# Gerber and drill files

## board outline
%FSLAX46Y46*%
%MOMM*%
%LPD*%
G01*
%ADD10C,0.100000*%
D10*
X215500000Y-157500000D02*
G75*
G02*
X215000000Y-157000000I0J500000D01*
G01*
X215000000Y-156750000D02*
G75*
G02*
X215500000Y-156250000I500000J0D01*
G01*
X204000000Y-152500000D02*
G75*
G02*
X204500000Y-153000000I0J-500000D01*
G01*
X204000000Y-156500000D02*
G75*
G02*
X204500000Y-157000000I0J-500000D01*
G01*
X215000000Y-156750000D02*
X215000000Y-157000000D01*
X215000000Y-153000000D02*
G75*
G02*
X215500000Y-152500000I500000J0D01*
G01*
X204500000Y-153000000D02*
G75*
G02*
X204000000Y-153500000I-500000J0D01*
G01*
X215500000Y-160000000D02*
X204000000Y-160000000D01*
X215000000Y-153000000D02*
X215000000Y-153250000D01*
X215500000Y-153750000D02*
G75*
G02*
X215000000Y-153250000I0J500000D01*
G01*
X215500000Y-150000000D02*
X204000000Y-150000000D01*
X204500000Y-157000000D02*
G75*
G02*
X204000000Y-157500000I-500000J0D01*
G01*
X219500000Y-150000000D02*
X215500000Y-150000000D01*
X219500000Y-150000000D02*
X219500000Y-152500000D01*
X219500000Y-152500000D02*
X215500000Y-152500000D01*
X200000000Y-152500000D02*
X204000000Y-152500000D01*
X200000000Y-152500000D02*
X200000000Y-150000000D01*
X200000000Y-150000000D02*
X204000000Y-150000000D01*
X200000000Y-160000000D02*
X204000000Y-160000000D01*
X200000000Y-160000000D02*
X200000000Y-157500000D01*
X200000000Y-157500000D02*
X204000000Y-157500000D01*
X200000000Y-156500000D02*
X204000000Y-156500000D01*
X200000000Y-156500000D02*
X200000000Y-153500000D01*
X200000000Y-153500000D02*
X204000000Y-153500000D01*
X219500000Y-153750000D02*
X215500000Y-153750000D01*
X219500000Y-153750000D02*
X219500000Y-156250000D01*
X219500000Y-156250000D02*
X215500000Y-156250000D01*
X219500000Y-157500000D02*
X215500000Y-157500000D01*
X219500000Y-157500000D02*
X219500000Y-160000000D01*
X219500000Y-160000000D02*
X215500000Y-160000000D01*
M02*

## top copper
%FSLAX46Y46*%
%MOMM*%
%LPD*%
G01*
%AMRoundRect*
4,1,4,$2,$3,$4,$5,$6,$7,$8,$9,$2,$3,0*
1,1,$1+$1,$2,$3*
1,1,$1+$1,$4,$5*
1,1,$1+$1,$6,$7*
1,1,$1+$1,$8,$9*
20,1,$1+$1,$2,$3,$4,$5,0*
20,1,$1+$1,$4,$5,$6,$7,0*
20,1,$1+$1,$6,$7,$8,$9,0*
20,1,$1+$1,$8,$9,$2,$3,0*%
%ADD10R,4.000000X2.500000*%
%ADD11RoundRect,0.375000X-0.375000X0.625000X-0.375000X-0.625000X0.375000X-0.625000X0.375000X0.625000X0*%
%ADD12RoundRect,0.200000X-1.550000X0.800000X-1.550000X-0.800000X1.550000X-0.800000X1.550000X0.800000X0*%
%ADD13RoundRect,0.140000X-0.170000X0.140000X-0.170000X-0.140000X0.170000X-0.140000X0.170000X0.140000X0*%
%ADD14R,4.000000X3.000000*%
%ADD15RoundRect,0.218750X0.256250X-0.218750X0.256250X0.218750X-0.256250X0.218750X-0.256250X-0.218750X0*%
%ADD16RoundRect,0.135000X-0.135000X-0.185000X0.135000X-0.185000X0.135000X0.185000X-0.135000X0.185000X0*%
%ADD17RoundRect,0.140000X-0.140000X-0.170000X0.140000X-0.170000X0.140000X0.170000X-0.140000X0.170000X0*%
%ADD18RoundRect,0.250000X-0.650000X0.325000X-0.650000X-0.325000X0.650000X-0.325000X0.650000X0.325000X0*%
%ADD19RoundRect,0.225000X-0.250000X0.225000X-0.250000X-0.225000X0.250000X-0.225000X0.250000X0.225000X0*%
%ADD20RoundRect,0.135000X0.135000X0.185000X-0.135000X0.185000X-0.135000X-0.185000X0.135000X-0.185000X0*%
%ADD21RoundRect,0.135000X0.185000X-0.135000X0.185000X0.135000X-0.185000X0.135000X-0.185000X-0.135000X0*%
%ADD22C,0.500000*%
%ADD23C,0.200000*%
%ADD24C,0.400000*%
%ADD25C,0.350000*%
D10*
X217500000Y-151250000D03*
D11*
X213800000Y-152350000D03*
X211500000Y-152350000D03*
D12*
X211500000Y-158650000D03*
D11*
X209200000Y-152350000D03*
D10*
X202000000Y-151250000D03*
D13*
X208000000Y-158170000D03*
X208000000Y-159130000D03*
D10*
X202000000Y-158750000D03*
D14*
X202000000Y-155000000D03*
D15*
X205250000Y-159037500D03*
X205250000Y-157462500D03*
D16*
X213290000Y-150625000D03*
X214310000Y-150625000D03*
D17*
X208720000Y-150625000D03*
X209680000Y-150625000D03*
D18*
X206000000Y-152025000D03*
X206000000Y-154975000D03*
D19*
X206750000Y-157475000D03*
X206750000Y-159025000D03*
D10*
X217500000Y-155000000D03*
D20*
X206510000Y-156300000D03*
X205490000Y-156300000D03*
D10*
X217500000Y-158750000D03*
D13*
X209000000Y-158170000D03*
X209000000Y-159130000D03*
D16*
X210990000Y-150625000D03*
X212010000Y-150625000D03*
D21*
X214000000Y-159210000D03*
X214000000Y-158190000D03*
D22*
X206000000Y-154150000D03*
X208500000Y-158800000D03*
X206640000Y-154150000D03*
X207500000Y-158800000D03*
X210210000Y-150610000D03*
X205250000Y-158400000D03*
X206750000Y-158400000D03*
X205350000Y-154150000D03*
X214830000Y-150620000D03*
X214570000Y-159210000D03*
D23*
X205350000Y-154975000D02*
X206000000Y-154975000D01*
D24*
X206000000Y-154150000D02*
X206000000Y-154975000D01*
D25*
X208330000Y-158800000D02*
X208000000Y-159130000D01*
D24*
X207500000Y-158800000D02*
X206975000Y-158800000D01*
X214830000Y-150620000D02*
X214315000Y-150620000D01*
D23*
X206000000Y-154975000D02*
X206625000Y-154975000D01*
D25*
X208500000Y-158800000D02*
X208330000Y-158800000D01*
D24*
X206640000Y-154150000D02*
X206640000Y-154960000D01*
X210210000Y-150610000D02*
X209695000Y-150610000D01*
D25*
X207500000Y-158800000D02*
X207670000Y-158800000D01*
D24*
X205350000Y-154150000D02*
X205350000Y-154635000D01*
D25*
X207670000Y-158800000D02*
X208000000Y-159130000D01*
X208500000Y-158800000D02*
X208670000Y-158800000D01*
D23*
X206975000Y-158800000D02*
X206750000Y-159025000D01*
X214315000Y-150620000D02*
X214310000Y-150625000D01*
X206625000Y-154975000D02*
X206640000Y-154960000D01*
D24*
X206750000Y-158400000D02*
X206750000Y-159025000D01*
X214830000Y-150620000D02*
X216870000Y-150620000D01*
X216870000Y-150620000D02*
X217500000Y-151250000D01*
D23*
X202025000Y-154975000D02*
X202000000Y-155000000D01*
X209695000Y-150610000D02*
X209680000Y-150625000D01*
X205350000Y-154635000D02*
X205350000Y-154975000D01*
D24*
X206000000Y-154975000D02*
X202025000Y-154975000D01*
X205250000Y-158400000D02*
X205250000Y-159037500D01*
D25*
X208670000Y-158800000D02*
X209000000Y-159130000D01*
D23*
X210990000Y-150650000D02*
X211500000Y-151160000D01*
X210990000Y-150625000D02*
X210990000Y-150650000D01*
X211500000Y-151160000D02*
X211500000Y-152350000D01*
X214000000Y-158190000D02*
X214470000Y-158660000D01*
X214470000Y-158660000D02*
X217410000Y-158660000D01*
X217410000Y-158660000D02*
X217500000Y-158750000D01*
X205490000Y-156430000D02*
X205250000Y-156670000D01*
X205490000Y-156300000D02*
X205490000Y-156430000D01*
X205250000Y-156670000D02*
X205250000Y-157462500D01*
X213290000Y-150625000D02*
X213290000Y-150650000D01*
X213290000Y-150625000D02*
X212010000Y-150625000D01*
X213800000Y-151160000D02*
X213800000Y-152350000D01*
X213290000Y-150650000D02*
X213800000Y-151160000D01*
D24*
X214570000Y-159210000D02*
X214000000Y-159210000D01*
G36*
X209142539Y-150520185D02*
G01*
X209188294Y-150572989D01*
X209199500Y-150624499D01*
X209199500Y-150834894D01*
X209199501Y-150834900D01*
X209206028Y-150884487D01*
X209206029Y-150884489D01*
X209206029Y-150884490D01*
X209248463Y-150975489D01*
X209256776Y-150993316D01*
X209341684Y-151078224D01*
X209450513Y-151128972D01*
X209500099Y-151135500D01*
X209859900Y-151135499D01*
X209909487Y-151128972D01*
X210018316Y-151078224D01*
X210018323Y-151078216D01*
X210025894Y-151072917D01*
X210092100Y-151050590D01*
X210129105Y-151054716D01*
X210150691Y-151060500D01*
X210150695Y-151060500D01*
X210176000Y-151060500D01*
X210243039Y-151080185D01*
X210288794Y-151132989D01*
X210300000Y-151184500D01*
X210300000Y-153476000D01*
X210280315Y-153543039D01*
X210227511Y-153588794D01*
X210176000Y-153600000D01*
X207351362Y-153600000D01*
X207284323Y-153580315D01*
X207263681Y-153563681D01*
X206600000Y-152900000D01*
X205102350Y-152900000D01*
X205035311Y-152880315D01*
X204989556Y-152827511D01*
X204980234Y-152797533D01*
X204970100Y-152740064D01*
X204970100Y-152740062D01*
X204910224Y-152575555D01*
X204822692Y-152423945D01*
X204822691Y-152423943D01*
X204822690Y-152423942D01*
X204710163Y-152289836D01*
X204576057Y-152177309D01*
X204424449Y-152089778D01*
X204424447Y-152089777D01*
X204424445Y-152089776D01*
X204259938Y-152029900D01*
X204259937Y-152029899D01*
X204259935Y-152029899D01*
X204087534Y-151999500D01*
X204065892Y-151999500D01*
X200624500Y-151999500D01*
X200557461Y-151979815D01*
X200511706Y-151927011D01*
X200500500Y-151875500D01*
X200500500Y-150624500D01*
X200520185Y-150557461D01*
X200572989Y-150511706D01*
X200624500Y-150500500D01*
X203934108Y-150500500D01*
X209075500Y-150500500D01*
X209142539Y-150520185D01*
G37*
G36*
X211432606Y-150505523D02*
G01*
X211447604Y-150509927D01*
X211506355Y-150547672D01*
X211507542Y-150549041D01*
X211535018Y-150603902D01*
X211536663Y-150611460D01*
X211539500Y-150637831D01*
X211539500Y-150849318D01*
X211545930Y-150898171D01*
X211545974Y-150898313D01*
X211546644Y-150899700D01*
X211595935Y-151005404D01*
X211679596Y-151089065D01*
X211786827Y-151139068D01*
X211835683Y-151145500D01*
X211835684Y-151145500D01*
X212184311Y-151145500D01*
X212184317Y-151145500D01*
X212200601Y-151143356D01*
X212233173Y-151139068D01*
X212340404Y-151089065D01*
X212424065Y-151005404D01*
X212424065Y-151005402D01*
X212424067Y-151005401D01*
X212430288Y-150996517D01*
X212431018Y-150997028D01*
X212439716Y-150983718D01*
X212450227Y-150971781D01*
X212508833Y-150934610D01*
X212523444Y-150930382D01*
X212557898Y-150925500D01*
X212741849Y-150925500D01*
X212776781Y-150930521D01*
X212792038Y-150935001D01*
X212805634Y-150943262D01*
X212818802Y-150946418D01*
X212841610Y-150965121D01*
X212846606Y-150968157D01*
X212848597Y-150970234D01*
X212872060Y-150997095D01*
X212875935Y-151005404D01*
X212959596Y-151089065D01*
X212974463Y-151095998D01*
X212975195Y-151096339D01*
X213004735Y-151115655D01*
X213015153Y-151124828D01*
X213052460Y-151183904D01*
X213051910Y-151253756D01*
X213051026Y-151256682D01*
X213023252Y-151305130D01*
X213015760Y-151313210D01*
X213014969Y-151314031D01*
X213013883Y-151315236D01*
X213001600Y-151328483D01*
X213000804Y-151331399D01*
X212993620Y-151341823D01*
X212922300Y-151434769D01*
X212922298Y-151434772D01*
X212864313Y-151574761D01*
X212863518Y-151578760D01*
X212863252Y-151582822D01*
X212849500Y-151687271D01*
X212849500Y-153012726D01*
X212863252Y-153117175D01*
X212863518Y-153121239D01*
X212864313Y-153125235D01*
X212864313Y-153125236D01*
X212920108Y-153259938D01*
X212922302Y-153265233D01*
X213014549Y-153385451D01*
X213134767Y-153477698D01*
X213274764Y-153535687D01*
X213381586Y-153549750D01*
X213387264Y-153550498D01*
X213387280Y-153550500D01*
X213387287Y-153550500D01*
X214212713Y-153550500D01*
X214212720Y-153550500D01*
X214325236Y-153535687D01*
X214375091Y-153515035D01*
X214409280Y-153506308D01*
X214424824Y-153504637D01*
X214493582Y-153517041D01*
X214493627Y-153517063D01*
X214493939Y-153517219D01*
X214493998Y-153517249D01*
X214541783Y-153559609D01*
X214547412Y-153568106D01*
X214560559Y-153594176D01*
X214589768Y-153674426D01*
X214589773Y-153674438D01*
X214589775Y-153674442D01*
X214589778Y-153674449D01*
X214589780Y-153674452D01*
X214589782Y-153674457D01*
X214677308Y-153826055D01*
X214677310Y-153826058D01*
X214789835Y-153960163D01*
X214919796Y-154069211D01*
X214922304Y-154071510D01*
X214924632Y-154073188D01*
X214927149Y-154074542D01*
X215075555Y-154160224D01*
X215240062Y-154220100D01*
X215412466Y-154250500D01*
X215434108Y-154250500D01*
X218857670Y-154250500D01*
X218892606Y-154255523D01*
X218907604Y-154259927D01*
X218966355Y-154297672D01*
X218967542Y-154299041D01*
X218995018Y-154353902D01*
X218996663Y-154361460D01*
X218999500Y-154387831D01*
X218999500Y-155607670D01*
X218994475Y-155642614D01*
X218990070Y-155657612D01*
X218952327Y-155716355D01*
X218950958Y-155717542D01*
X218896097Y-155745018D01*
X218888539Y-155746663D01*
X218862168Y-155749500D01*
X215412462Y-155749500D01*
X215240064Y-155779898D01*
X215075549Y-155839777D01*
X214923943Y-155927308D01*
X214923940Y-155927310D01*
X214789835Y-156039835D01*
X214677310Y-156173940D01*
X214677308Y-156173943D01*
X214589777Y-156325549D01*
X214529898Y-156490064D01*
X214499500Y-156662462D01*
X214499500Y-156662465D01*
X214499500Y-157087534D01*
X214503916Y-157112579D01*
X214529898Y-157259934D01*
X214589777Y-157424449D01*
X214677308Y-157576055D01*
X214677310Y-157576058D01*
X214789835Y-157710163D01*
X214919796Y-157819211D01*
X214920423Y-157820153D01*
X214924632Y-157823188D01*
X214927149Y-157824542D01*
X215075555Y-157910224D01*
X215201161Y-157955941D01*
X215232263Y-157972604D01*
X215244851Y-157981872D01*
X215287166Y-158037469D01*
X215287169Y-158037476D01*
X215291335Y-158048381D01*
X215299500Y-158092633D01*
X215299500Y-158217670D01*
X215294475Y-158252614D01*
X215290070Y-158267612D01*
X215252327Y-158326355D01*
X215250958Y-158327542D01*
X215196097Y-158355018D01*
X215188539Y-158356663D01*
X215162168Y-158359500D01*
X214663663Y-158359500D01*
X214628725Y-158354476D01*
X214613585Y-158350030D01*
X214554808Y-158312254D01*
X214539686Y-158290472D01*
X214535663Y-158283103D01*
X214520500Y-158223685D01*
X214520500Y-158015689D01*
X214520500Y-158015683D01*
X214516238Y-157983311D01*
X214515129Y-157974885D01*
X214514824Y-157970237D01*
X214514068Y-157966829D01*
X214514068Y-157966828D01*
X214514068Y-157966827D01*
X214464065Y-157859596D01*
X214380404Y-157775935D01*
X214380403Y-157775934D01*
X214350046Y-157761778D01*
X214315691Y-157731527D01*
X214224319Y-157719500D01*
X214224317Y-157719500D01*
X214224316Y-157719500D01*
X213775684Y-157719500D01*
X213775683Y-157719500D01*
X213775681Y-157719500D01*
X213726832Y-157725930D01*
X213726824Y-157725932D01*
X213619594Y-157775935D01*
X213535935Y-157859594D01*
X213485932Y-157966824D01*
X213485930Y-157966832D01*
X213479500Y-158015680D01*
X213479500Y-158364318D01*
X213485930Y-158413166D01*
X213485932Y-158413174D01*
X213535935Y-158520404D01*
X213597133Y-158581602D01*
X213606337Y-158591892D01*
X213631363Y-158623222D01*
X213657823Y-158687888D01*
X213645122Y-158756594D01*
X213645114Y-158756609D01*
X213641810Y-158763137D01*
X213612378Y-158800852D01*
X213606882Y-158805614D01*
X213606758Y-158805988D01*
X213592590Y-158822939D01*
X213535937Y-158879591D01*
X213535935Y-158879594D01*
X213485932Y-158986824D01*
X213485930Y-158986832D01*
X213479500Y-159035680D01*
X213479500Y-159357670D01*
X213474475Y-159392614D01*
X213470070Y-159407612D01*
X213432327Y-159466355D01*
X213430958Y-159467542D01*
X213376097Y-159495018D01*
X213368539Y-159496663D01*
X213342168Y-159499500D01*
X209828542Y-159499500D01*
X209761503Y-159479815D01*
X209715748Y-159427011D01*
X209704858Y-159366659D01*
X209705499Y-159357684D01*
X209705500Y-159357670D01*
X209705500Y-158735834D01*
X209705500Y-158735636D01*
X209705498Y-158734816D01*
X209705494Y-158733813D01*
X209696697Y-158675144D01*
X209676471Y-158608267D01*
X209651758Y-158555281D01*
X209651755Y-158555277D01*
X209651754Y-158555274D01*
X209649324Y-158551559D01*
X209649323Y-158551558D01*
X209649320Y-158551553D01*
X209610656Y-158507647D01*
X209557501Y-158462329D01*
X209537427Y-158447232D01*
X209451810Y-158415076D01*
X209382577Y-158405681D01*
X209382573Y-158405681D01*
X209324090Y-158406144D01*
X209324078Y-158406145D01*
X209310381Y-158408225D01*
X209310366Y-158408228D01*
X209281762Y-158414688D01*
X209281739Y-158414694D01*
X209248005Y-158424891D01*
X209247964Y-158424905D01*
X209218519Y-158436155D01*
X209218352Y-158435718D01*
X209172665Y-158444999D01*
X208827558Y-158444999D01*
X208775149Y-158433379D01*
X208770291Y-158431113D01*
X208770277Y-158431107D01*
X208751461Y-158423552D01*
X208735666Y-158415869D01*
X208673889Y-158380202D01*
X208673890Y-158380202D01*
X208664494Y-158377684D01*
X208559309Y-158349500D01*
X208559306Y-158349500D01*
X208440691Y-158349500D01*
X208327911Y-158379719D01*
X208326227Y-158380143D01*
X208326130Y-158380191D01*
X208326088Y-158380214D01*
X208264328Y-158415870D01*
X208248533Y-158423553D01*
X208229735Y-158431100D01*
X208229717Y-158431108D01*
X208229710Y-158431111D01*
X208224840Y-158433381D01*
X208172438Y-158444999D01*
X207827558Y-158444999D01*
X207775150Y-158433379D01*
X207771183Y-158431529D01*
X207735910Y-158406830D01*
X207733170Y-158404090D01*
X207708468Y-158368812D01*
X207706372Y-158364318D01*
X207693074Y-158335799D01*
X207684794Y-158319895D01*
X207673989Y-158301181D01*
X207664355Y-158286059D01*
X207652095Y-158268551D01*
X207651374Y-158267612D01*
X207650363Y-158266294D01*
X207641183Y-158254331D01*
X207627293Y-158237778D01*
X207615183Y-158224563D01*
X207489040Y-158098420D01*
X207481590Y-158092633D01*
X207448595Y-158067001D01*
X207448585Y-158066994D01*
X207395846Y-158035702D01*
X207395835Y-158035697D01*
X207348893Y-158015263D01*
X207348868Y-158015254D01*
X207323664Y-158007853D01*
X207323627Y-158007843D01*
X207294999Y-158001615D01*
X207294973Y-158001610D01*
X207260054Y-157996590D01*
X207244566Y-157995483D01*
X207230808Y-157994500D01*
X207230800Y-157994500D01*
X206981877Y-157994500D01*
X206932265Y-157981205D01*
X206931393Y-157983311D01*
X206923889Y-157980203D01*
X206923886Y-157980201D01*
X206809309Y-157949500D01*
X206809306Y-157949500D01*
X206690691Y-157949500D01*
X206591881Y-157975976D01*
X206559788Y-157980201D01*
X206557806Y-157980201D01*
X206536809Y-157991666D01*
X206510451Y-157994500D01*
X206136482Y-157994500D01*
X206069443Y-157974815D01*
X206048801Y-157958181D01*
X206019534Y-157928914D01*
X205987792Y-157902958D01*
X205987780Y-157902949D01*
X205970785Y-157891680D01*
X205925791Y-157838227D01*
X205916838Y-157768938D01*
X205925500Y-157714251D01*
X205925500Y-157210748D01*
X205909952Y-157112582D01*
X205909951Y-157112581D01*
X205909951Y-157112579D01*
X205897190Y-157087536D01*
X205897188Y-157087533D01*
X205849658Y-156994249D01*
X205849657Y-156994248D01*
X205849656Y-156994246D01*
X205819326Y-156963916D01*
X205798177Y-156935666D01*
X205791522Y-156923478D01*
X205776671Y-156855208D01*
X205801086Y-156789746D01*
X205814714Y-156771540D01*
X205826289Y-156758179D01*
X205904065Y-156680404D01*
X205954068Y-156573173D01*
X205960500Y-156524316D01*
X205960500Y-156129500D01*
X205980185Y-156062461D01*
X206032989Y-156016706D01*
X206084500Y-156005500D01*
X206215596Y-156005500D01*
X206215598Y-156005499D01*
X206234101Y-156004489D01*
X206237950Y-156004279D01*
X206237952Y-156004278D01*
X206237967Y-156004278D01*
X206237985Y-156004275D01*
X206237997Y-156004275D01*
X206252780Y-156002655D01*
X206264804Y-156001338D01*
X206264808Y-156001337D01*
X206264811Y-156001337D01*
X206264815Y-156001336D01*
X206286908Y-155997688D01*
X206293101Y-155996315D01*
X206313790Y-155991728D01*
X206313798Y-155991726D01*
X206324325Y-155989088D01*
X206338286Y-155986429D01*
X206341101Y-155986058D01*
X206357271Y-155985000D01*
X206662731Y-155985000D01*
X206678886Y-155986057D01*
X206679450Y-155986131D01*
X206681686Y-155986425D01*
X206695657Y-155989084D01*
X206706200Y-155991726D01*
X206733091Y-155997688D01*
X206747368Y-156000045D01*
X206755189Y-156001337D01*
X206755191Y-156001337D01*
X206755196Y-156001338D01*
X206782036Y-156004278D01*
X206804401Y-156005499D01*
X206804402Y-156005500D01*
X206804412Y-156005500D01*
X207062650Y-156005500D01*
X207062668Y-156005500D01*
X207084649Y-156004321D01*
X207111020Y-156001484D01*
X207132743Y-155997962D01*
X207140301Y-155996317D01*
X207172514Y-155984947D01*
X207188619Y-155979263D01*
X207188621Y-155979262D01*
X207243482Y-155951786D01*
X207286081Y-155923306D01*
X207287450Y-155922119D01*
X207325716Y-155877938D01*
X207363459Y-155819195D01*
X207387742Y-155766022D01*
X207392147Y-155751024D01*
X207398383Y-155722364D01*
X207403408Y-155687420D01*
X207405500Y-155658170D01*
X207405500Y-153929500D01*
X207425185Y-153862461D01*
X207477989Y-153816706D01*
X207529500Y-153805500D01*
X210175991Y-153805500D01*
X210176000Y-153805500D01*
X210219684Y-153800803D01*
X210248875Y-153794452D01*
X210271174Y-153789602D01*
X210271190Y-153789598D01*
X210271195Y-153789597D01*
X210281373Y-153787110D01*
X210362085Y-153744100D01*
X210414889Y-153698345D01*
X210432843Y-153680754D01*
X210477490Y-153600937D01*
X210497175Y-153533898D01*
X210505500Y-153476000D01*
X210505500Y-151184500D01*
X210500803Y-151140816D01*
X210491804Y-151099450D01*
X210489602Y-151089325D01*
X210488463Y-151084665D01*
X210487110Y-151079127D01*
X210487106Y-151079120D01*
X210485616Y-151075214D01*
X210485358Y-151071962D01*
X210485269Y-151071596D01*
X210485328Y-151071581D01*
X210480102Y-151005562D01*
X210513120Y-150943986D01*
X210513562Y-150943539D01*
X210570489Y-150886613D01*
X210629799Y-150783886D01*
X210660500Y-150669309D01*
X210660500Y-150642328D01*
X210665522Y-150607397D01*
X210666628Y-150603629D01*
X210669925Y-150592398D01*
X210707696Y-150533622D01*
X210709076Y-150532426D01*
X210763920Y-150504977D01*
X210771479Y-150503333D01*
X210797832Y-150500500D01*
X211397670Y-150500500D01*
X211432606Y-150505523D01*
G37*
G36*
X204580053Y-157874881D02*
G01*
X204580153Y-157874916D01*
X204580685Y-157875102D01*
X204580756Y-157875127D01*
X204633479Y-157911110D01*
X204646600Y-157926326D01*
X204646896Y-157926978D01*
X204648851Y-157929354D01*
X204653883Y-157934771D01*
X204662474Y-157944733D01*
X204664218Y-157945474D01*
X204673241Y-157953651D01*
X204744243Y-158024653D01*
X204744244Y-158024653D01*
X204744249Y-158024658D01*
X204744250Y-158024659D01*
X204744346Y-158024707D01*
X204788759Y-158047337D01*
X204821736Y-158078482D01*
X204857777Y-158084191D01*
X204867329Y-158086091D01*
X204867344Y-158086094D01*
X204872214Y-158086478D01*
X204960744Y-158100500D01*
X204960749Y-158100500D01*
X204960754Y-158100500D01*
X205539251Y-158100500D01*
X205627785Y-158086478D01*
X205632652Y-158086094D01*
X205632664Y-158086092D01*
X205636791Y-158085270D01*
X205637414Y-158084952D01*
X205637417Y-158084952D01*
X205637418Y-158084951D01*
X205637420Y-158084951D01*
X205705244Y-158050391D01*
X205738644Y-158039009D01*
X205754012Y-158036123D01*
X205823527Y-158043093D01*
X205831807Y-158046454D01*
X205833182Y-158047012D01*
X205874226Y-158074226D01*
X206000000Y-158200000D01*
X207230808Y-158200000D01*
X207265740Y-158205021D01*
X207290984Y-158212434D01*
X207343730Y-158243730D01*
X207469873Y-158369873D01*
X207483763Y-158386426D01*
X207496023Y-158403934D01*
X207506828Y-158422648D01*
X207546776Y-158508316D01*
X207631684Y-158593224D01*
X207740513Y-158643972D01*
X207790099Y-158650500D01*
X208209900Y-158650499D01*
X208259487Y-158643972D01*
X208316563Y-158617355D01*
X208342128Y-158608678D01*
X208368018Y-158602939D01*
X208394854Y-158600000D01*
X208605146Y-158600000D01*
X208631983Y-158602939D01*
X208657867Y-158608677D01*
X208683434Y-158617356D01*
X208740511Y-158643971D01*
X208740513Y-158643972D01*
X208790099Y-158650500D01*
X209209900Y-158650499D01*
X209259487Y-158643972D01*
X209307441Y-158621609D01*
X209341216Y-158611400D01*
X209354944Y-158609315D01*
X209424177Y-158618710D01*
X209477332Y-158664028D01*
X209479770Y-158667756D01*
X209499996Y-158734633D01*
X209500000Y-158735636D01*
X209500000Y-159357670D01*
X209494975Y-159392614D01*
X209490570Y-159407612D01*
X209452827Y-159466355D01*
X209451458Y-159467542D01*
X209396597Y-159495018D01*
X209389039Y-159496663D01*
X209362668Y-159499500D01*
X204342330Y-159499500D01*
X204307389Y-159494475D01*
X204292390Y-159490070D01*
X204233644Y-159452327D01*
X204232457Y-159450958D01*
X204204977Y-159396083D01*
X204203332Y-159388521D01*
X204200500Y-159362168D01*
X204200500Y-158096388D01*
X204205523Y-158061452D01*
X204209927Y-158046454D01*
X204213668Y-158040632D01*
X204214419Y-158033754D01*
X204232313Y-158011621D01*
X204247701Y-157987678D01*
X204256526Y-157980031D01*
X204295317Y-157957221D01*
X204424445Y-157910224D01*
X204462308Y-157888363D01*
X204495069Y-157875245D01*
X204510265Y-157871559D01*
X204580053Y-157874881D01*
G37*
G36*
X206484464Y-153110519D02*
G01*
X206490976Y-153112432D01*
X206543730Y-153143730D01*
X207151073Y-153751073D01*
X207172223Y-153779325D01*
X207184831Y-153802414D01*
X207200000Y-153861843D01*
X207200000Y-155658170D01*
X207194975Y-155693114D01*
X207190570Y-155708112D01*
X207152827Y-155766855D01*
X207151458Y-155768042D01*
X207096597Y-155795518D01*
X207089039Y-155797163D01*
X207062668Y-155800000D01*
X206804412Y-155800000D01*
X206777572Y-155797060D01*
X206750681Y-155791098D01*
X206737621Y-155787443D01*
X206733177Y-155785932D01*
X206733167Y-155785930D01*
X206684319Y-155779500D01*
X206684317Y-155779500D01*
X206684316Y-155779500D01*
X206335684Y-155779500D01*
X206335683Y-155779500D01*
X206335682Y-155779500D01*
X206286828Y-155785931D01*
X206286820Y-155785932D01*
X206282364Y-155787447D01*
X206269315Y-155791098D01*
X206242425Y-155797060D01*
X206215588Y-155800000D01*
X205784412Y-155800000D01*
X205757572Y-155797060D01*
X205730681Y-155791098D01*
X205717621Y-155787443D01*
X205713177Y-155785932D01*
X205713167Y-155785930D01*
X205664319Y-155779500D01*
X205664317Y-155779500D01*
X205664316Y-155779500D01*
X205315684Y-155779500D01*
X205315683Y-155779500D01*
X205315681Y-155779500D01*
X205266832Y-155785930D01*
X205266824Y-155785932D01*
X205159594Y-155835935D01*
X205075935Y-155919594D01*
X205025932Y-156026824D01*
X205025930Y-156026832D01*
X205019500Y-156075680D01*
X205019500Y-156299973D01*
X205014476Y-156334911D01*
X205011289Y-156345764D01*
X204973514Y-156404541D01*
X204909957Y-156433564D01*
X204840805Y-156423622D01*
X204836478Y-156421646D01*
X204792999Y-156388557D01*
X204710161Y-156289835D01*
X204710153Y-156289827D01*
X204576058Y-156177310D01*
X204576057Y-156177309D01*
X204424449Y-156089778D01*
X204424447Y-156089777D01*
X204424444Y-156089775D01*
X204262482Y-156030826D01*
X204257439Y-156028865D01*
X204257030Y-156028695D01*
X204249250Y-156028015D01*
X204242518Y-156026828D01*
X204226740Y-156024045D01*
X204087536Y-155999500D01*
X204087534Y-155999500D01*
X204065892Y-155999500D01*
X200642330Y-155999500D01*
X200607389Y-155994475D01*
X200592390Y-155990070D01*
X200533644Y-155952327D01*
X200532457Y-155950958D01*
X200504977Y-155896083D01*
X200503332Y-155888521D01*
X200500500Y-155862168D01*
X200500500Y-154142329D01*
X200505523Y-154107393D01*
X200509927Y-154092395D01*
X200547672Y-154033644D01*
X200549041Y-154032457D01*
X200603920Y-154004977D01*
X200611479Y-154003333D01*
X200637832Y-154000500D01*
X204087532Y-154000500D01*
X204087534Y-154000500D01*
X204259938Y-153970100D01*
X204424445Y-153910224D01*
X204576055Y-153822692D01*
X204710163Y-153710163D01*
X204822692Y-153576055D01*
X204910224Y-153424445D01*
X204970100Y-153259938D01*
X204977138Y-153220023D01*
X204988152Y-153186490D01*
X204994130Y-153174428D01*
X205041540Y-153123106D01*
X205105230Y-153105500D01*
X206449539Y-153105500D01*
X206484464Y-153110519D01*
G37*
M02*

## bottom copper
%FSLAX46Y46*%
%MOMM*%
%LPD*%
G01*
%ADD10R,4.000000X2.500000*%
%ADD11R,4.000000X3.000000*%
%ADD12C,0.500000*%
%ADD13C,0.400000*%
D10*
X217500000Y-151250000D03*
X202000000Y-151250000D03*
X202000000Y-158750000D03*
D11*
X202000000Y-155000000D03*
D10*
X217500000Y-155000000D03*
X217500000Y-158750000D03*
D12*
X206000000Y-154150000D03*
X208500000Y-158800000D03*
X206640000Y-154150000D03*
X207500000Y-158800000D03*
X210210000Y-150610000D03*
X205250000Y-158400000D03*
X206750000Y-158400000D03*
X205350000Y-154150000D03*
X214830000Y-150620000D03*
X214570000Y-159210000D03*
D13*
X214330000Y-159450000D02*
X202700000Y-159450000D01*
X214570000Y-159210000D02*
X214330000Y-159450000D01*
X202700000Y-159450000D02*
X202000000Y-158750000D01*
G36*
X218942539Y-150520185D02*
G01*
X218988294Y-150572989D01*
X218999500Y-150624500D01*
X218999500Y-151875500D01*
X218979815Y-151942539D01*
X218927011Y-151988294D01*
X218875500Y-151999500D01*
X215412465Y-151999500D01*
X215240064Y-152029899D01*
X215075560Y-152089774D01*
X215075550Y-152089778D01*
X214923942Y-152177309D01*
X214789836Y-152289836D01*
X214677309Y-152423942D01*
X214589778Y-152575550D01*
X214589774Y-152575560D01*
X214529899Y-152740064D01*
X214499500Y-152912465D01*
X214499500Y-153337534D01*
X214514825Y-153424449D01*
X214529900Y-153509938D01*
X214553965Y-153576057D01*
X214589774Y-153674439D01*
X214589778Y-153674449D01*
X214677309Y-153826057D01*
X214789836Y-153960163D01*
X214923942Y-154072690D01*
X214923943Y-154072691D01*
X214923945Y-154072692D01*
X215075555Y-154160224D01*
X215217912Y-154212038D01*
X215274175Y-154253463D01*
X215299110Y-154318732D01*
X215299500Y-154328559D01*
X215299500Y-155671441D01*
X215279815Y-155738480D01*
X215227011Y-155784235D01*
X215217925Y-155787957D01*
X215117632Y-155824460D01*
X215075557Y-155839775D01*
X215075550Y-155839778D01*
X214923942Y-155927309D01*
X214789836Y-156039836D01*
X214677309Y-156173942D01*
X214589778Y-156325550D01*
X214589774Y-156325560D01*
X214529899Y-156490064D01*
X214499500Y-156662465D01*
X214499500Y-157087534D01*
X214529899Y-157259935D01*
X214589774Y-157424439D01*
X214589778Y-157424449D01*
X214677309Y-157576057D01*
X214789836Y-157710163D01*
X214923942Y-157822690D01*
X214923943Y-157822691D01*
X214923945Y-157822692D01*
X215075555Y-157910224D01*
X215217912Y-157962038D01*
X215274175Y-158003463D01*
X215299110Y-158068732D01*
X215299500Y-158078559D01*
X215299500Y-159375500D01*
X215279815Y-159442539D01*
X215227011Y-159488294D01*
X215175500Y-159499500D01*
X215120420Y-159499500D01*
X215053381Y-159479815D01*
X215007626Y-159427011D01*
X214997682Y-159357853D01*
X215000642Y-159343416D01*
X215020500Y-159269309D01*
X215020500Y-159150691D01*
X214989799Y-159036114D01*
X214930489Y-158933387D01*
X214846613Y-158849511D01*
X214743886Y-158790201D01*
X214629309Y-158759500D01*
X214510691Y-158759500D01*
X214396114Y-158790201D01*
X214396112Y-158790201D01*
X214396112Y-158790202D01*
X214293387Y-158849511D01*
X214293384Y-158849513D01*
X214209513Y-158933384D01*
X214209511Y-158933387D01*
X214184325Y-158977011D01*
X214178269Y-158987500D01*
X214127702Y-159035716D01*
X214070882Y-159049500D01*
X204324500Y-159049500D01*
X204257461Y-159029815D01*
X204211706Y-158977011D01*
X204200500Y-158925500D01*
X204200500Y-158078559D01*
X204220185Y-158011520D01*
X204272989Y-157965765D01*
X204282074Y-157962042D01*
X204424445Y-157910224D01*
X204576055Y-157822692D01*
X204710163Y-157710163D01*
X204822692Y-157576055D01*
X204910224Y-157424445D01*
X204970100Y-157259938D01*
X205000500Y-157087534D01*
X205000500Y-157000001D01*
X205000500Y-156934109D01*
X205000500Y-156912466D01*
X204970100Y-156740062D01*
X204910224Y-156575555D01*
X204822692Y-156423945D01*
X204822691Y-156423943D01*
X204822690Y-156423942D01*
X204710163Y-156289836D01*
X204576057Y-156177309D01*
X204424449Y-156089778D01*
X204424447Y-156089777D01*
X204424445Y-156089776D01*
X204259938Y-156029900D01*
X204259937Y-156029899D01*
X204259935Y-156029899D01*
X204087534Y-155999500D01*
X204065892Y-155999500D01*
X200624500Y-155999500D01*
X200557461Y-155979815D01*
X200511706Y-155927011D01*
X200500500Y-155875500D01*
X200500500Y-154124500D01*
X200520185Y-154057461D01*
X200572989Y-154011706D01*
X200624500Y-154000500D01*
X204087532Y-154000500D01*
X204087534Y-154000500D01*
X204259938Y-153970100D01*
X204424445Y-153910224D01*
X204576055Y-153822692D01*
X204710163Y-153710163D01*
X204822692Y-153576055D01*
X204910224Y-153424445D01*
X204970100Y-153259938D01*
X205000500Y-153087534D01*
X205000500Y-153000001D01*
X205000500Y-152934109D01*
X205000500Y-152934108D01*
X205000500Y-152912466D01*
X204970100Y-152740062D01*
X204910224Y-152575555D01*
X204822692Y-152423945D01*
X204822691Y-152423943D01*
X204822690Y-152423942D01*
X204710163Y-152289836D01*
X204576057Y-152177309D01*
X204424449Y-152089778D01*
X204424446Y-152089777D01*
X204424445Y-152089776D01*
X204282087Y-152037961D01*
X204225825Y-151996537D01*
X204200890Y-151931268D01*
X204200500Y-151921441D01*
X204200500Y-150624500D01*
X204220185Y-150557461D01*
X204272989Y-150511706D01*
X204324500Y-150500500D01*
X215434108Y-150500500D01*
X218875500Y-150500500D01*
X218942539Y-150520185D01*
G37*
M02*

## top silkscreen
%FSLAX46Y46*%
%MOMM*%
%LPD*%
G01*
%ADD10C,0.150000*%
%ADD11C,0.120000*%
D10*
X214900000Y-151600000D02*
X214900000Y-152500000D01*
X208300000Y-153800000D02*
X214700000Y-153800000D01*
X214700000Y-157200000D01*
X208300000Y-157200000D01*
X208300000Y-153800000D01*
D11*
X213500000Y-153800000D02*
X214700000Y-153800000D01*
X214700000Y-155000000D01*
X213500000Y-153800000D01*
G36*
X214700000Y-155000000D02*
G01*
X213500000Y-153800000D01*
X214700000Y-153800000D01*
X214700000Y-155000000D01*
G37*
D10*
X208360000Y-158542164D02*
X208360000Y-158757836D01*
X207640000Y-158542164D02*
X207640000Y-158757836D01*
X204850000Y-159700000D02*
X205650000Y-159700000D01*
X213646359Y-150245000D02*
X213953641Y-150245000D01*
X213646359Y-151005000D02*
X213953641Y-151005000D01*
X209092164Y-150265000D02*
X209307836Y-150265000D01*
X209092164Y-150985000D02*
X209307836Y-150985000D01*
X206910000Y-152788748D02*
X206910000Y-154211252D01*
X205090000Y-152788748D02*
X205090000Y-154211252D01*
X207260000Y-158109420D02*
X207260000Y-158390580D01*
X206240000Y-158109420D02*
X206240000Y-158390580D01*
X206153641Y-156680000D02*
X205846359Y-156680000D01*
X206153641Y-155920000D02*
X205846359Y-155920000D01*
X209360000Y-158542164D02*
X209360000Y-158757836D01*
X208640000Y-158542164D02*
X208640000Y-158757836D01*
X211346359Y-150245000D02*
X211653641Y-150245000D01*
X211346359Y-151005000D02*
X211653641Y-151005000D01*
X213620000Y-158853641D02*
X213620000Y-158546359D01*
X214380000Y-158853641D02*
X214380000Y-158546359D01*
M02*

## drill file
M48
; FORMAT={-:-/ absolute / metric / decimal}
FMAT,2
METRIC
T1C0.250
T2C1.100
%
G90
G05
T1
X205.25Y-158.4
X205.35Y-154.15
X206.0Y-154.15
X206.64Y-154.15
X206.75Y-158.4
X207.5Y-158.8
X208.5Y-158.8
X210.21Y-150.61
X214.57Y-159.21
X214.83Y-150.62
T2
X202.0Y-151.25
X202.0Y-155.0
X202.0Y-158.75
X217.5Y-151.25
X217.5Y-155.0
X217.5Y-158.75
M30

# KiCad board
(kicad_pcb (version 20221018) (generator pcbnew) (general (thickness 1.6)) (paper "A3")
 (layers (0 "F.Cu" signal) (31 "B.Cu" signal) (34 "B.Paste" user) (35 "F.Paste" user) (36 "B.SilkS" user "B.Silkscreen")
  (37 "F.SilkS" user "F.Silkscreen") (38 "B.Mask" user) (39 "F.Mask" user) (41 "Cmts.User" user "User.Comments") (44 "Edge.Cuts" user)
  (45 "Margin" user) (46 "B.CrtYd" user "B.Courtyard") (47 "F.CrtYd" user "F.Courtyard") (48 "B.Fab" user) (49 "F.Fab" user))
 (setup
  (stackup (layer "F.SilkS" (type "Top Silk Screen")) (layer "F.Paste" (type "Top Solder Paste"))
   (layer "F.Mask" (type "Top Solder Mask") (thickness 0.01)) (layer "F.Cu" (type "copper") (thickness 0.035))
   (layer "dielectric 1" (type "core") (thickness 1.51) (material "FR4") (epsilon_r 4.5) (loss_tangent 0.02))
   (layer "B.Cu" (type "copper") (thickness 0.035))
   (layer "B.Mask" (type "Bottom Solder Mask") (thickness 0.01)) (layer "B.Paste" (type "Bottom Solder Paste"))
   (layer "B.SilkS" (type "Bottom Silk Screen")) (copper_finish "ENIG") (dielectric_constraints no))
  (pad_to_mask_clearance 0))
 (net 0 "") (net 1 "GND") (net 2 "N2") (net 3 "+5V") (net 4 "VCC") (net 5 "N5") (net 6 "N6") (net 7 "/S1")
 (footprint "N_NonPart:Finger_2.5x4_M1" (layer "F.Cu") (at 217.5 151.25)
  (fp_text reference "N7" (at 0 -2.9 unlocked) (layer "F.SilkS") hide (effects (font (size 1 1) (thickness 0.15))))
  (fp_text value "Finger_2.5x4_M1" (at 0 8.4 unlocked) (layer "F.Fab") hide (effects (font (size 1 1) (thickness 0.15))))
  (fp_line (start 2 -1.25) (end -2 -1.25) (stroke (width 0.1) (type solid)) (layer "Edge.Cuts"))
  (fp_line (start 2 -1.25) (end 2 1.25) (stroke (width 0.1) (type default)) (layer "Edge.Cuts"))
  (fp_line (start 2 1.25) (end -2 1.25) (stroke (width 0.1) (type solid)) (layer "Edge.Cuts"))
  (pad "1" thru_hole rect (at 0 0) (size 4 2.5) (drill 1.1) (layers "*.Cu" "*.Mask") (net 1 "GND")))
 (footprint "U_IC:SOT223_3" (layer "F.Cu") (at 211.5 155.5 -90)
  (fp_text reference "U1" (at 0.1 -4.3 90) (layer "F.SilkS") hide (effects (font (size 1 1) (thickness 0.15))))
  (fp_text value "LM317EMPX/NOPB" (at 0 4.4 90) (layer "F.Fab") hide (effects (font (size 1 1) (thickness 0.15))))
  (fp_line (start -3.9 -3.4) (end -3 -3.4) (stroke (width 0.15) (type solid)) (layer "F.SilkS"))
  (fp_rect (start -1.7 3.2) (end 1.7 -3.2) (stroke (width 0.15) (type solid)) (fill none) (layer "F.SilkS"))
  (fp_poly (pts (xy -1.7 -2) (xy -1.7 -3.2) (xy -0.5 -3.2)) (stroke (width 0.12) (type solid)) (fill solid) (layer "F.SilkS"))
  (pad "1" smd roundrect (at -3.15 -2.3 270) (size 2 1.5) (layers "F.Cu" "F.Paste" "F.Mask") (roundrect_rratio 0.25) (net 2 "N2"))
  (pad "2" smd roundrect (at -3.15 0 270) (size 2 1.5) (layers "F.Cu" "F.Paste" "F.Mask") (roundrect_rratio 0.25) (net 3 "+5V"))
  (pad "2" smd roundrect (at 3.15 0 270) (size 2 3.5) (layers "F.Cu" "F.Paste" "F.Mask") (roundrect_rratio 0.1) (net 3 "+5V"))
  (pad "3" smd roundrect (at -3.15 2.3 270) (size 2 1.5) (layers "F.Cu" "F.Paste" "F.Mask") (roundrect_rratio 0.25) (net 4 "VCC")))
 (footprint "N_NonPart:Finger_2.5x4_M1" (layer "F.Cu") (at 202 151.25 180)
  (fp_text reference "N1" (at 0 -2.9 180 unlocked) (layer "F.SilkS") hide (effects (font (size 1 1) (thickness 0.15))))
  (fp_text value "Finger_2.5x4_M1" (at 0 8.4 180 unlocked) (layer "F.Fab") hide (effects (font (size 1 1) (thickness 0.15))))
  (fp_line (start 2 -1.25) (end -2 -1.25) (stroke (width 0.1) (type solid)) (layer "Edge.Cuts"))
  (fp_line (start 2 -1.25) (end 2 1.25) (stroke (width 0.1) (type default)) (layer "Edge.Cuts"))
  (fp_line (start 2 1.25) (end -2 1.25) (stroke (width 0.1) (type solid)) (layer "Edge.Cuts"))
  (pad "1" thru_hole rect (at 0 0 180) (size 4 2.5) (drill 1.1) (layers "*.Cu" "*.Mask") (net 4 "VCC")))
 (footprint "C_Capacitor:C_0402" (layer "F.Cu") (at 208 158.65 -90)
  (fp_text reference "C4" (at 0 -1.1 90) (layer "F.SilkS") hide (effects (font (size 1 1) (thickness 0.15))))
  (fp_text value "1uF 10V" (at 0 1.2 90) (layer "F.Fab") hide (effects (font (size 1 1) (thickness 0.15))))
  (fp_line (start -0.107836 -0.36) (end 0.107836 -0.36) (stroke (width 0.15) (type solid)) (layer "F.SilkS"))
  (fp_line (start -0.107836 0.36) (end 0.107836 0.36) (stroke (width 0.15) (type solid)) (layer "F.SilkS"))
  (pad "1" smd roundrect (at -0.48 0 270) (size 0.56 0.62) (layers "F.Cu" "F.Paste" "F.Mask") (roundrect_rratio 0.25) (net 3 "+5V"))
  (pad "2" smd roundrect (at 0.48 0 270) (size 0.56 0.62) (layers "F.Cu" "F.Paste" "F.Mask") (roundrect_rratio 0.25) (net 1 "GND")))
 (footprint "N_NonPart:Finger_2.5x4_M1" (layer "F.Cu") (at 202 158.75 180)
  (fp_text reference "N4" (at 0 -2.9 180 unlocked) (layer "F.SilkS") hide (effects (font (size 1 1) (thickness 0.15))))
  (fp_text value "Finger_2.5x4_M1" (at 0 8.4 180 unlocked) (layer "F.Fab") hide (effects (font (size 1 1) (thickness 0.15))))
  (fp_line (start 2 -1.25) (end -2 -1.25) (stroke (width 0.1) (type solid)) (layer "Edge.Cuts"))
  (fp_line (start 2 -1.25) (end 2 1.25) (stroke (width 0.1) (type default)) (layer "Edge.Cuts"))
  (fp_line (start 2 1.25) (end -2 1.25) (stroke (width 0.1) (type solid)) (layer "Edge.Cuts"))
  (pad "1" thru_hole rect (at 0 0 180) (size 4 2.5) (drill 1.1) (layers "*.Cu" "*.Mask") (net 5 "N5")))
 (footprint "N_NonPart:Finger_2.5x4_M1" (layer "F.Cu") (at 202 155 180)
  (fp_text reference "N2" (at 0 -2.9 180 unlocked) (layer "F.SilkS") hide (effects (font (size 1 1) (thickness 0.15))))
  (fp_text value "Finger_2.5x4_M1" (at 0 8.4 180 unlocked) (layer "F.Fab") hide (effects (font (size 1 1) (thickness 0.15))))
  (fp_line (start 2 -1.5) (end -2 -1.5) (stroke (width 0.1) (type solid)) (layer "Edge.Cuts"))
  (fp_line (start 2 -1.5) (end 2 1.5) (stroke (width 0.1) (type default)) (layer "Edge.Cuts"))
  (fp_line (start 2 1.5) (end -2 1.5) (stroke (width 0.1) (type solid)) (layer "Edge.Cuts"))
  (pad "1" thru_hole rect (at 0 0 180) (size 4 3) (drill 1.1) (layers "*.Cu" "*.Mask") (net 1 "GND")))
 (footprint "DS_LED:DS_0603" (layer "F.Cu") (at 205.25 158.25 90)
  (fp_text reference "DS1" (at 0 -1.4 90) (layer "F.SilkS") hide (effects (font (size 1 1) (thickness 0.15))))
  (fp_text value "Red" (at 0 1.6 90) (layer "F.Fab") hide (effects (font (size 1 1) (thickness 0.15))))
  (fp_line (start -1.45 -0.4) (end -1.45 0.4) (stroke (width 0.15) (type solid)) (layer "F.SilkS"))
  (pad "1" smd roundrect (at -0.7875 0 90) (size 0.875 0.95) (layers "F.Cu" "F.Paste" "F.Mask") (roundrect_rratio 0.25) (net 1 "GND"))
  (pad "2" smd roundrect (at 0.7875 0 90) (size 0.875 0.95) (layers "F.Cu" "F.Paste" "F.Mask") (roundrect_rratio 0.25) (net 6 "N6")))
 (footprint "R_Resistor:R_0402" (layer "F.Cu") (at 213.8 150.625)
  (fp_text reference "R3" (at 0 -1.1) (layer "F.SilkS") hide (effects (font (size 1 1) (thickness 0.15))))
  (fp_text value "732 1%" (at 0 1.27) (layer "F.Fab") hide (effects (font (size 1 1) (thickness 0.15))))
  (fp_line (start -0.153641 -0.38) (end 0.153641 -0.38) (stroke (width 0.15) (type solid)) (layer "F.SilkS"))
  (fp_line (start -0.153641 0.38) (end 0.153641 0.38) (stroke (width 0.15) (type solid)) (layer "F.SilkS"))
  (pad "1" smd roundrect (at -0.51 0) (size 0.54 0.64) (layers "F.Cu" "F.Paste" "F.Mask") (roundrect_rratio 0.25) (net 2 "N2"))
  (pad "2" smd roundrect (at 0.51 0) (size 0.54 0.64) (layers "F.Cu" "F.Paste" "F.Mask") (roundrect_rratio 0.25) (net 1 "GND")))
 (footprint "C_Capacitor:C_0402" (layer "F.Cu") (at 209.2 150.625)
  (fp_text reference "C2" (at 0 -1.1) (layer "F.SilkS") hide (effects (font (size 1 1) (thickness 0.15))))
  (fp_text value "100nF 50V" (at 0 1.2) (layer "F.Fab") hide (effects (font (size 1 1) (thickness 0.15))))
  (fp_line (start -0.107836 -0.36) (end 0.107836 -0.36) (stroke (width 0.15) (type solid)) (layer "F.SilkS"))
  (fp_line (start -0.107836 0.36) (end 0.107836 0.36) (stroke (width 0.15) (type solid)) (layer "F.SilkS"))
  (pad "1" smd roundrect (at -0.48 0) (size 0.56 0.62) (layers "F.Cu" "F.Paste" "F.Mask") (roundrect_rratio 0.25) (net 4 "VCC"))
  (pad "2" smd roundrect (at 0.48 0) (size 0.56 0.62) (layers "F.Cu" "F.Paste" "F.Mask") (roundrect_rratio 0.25) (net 1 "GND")))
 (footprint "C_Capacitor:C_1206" (layer "F.Cu") (at 206 153.5 -90)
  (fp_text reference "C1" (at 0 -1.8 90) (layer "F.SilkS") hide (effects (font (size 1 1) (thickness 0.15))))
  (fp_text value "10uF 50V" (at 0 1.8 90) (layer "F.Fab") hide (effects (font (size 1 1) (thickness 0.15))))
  (fp_line (start -0.711252 -0.91) (end 0.711252 -0.91) (stroke (width 0.15) (type solid)) (layer "F.SilkS"))
  (fp_line (start -0.711252 0.91) (end 0.711252 0.91) (stroke (width 0.15) (type solid)) (layer "F.SilkS"))
  (pad "1" smd roundrect (at -1.475 0 270) (size 1.15 1.8) (layers "F.Cu" "F.Paste" "F.Mask") (roundrect_rratio 0.217391) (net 4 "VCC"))
  (pad "2" smd roundrect (at 1.475 0 270) (size 1.15 1.8) (layers "F.Cu" "F.Paste" "F.Mask") (roundrect_rratio 0.217391) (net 1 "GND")))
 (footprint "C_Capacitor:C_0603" (layer "F.Cu") (at 206.75 158.25 -90)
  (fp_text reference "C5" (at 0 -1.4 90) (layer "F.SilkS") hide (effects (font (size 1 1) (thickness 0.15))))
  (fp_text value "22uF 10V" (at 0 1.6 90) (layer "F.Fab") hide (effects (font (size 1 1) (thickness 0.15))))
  (fp_line (start -0.14058 -0.51) (end 0.14058 -0.51) (stroke (width 0.15) (type solid)) (layer "F.SilkS"))
  (fp_line (start -0.14058 0.51) (end 0.14058 0.51) (stroke (width 0.15) (type solid)) (layer "F.SilkS"))
  (pad "1" smd roundrect (at -0.775 0 270) (size 0.9 0.95) (layers "F.Cu" "F.Paste" "F.Mask") (roundrect_rratio 0.25) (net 3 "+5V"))
  (pad "2" smd roundrect (at 0.775 0 270) (size 0.9 0.95) (layers "F.Cu" "F.Paste" "F.Mask") (roundrect_rratio 0.25) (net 1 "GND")))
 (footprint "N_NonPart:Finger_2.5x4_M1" (layer "F.Cu") (at 217.5 155)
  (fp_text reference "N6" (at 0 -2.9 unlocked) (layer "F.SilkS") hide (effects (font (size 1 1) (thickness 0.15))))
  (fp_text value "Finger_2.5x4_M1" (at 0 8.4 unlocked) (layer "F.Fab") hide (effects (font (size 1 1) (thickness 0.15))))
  (fp_line (start 2 -1.25) (end -2 -1.25) (stroke (width 0.1) (type solid)) (layer "Edge.Cuts"))
  (fp_line (start 2 -1.25) (end 2 1.25) (stroke (width 0.1) (type default)) (layer "Edge.Cuts"))
  (fp_line (start 2 1.25) (end -2 1.25) (stroke (width 0.1) (type solid)) (layer "Edge.Cuts"))
  (pad "1" thru_hole rect (at 0 0) (size 4 2.5) (drill 1.1) (layers "*.Cu" "*.Mask") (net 3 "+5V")))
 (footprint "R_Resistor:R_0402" (layer "F.Cu") (at 206 156.3 180)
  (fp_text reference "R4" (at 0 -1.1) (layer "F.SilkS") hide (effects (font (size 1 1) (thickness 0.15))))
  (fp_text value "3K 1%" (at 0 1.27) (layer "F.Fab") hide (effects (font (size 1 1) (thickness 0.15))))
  (fp_line (start -0.153641 -0.38) (end 0.153641 -0.38) (stroke (width 0.15) (type solid)) (layer "F.SilkS"))
  (fp_line (start -0.153641 0.38) (end 0.153641 0.38) (stroke (width 0.15) (type solid)) (layer "F.SilkS"))
  (pad "1" smd roundrect (at -0.51 0 180) (size 0.54 0.64) (layers "F.Cu" "F.Paste" "F.Mask") (roundrect_rratio 0.25) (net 3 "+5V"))
  (pad "2" smd roundrect (at 0.51 0 180) (size 0.54 0.64) (layers "F.Cu" "F.Paste" "F.Mask") (roundrect_rratio 0.25) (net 6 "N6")))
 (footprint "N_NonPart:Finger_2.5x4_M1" (layer "F.Cu") (at 217.5 158.75)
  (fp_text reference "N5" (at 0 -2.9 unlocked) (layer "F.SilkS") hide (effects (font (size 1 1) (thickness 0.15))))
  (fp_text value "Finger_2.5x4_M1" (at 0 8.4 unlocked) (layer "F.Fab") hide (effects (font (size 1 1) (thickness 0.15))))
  (fp_line (start 2 -1.25) (end -2 -1.25) (stroke (width 0.1) (type solid)) (layer "Edge.Cuts"))
  (fp_line (start 2 -1.25) (end 2 1.25) (stroke (width 0.1) (type default)) (layer "Edge.Cuts"))
  (fp_line (start 2 1.25) (end -2 1.25) (stroke (width 0.1) (type solid)) (layer "Edge.Cuts"))
  (pad "1" thru_hole rect (at 0 0) (size 4 2.5) (drill 1.1) (layers "*.Cu" "*.Mask") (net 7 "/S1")))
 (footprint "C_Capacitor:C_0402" (layer "F.Cu") (at 209 158.65 -90)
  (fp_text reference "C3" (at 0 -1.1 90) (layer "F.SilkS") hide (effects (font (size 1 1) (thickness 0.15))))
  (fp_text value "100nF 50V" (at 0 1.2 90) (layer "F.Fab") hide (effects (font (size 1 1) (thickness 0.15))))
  (fp_line (start -0.107836 -0.36) (end 0.107836 -0.36) (stroke (width 0.15) (type solid)) (layer "F.SilkS"))
  (fp_line (start -0.107836 0.36) (end 0.107836 0.36) (stroke (width 0.15) (type solid)) (layer "F.SilkS"))
  (pad "1" smd roundrect (at -0.48 0 270) (size 0.56 0.62) (layers "F.Cu" "F.Paste" "F.Mask") (roundrect_rratio 0.25) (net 3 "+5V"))
  (pad "2" smd roundrect (at 0.48 0 270) (size 0.56 0.62) (layers "F.Cu" "F.Paste" "F.Mask") (roundrect_rratio 0.25) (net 1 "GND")))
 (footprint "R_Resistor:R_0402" (layer "F.Cu") (at 211.5 150.625)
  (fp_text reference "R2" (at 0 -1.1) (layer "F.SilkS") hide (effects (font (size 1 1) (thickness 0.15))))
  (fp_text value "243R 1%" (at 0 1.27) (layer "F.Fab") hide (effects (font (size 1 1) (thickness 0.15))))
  (fp_line (start -0.153641 -0.38) (end 0.153641 -0.38) (stroke (width 0.15) (type solid)) (layer "F.SilkS"))
  (fp_line (start -0.153641 0.38) (end 0.153641 0.38) (stroke (width 0.15) (type solid)) (layer "F.SilkS"))
  (pad "1" smd roundrect (at -0.51 0) (size 0.54 0.64) (layers "F.Cu" "F.Paste" "F.Mask") (roundrect_rratio 0.25) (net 3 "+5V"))
  (pad "2" smd roundrect (at 0.51 0) (size 0.54 0.64) (layers "F.Cu" "F.Paste" "F.Mask") (roundrect_rratio 0.25) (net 2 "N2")))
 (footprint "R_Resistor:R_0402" (layer "F.Cu") (at 214 158.7 90)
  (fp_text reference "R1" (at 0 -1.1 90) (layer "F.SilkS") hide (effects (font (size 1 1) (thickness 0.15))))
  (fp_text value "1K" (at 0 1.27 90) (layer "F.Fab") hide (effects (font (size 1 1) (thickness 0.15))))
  (fp_line (start -0.153641 -0.38) (end 0.153641 -0.38) (stroke (width 0.15) (type solid)) (layer "F.SilkS"))
  (fp_line (start -0.153641 0.38) (end 0.153641 0.38) (stroke (width 0.15) (type solid)) (layer "F.SilkS"))
  (pad "1" smd roundrect (at -0.51 0 90) (size 0.54 0.64) (layers "F.Cu" "F.Paste" "F.Mask") (roundrect_rratio 0.25) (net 5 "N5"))
  (pad "2" smd roundrect (at 0.51 0 90) (size 0.54 0.64) (layers "F.Cu" "F.Paste" "F.Mask") (roundrect_rratio 0.25) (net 7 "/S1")))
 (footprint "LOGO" (layer "B.Cu") (at 209.63 153.17 180)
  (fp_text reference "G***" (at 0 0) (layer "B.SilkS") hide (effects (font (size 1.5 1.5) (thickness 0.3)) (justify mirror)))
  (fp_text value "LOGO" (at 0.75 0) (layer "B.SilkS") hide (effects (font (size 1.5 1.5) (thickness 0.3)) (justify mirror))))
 (gr_arc (start 215.5 157.5) (mid 215.146447 157.353553) (end 215 157) (stroke (width 0.1) (type default)) (layer "Edge.Cuts"))
 (gr_arc (start 215 156.75) (mid 215.146447 156.396447) (end 215.5 156.25) (stroke (width 0.1) (type default)) (layer "Edge.Cuts"))
 (gr_arc (start 204 152.5) (mid 204.353553 152.646447) (end 204.5 153) (stroke (width 0.1) (type default)) (layer "Edge.Cuts"))
 (gr_arc (start 204 156.5) (mid 204.353553 156.646447) (end 204.5 157) (stroke (width 0.1) (type default)) (layer "Edge.Cuts"))
 (gr_line (start 215 156.75) (end 215 157) (stroke (width 0.1) (type default)) (layer "Edge.Cuts"))
 (gr_arc (start 215 153) (mid 215.146447 152.646447) (end 215.5 152.5) (stroke (width 0.1) (type default)) (layer "Edge.Cuts"))
 (gr_arc (start 204.5 153) (mid 204.353553 153.353553) (end 204 153.5) (stroke (width 0.1) (type default)) (layer "Edge.Cuts"))
 (gr_line (start 215.5 160) (end 204 160) (stroke (width 0.1) (type default)) (layer "Edge.Cuts"))
 (gr_line (start 215 153) (end 215 153.25) (stroke (width 0.1) (type default)) (layer "Edge.Cuts"))
 (gr_arc (start 215.5 153.75) (mid 215.146447 153.603553) (end 215 153.25) (stroke (width 0.1) (type default)) (layer "Edge.Cuts"))
 (gr_line (start 215.5 150) (end 204 150) (stroke (width 0.1) (type default)) (layer "Edge.Cuts"))
 (gr_arc (start 204.5 157) (mid 204.353553 157.353553) (end 204 157.5) (stroke (width 0.1) (type default)) (layer "Edge.Cuts"))
 (segment (start 205.35 154.975) (end 206 154.975) (width 0.2) (layer "F.Cu") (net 1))
 (segment (start 206 154.15) (end 206 154.975) (width 0.4) (layer "F.Cu") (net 1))
 (segment (start 208.33 158.8) (end 208 159.13) (width 0.35) (layer "F.Cu") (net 1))
 (segment (start 207.5 158.8) (end 206.975 158.8) (width 0.4) (layer "F.Cu") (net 1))
 (segment (start 214.83 150.62) (end 214.315 150.62) (width 0.4) (layer "F.Cu") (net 1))
 (segment (start 206 154.975) (end 206.625 154.975) (width 0.2) (layer "F.Cu") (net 1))
 (segment (start 208.5 158.8) (end 208.33 158.8) (width 0.35) (layer "F.Cu") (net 1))
 (segment (start 206.64 154.15) (end 206.64 154.96) (width 0.4) (layer "F.Cu") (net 1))
 (segment (start 210.21 150.61) (end 209.695 150.61) (width 0.4) (layer "F.Cu") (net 1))
 (segment (start 207.5 158.8) (end 207.67 158.8) (width 0.35) (layer "F.Cu") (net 1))
 (segment (start 205.35 154.15) (end 205.35 154.635) (width 0.4) (layer "F.Cu") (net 1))
 (segment (start 207.67 158.8) (end 208 159.13) (width 0.35) (layer "F.Cu") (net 1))
 (segment (start 208.5 158.8) (end 208.67 158.8) (width 0.35) (layer "F.Cu") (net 1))
 (segment (start 206.975 158.8) (end 206.75 159.025) (width 0.2) (layer "F.Cu") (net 1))
 (segment (start 214.315 150.62) (end 214.31 150.625) (width 0.2) (layer "F.Cu") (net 1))
 (segment (start 206.625 154.975) (end 206.64 154.96) (width 0.2) (layer "F.Cu") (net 1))
 (segment (start 206.75 158.4) (end 206.75 159.025) (width 0.4) (layer "F.Cu") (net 1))
 (segment (start 214.83 150.62) (end 216.87 150.62) (width 0.4) (layer "F.Cu") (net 1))
 (segment (start 216.87 150.62) (end 217.5 151.25) (width 0.4) (layer "F.Cu") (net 1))
 (segment (start 202.025 154.975) (end 202 155) (width 0.2) (layer "F.Cu") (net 1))
 (segment (start 209.695 150.61) (end 209.68 150.625) (width 0.2) (layer "F.Cu") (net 1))
 (segment (start 205.35 154.635) (end 205.35 154.975) (width 0.2) (layer "F.Cu") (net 1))
 (segment (start 206 154.975) (end 202.025 154.975) (width 0.4) (layer "F.Cu") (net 1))
 (segment (start 205.25 158.4) (end 205.25 159.0375) (width 0.4) (layer "F.Cu") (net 1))
 (segment (start 208.67 158.8) (end 209 159.13) (width 0.35) (layer "F.Cu") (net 1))
 (via (at 206 154.15) (size 0.5) (drill 0.25) (layers "F.Cu" "B.Cu") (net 1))
 (via (at 208.5 158.8) (size 0.5) (drill 0.25) (layers "F.Cu" "B.Cu") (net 1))
 (via (at 206.64 154.15) (size 0.5) (drill 0.25) (layers "F.Cu" "B.Cu") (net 1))
 (via (at 207.5 158.8) (size 0.5) (drill 0.25) (layers "F.Cu" "B.Cu") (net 1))
 (via (at 210.21 150.61) (size 0.5) (drill 0.25) (layers "F.Cu" "B.Cu") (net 1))
 (via (at 205.25 158.4) (size 0.5) (drill 0.25) (layers "F.Cu" "B.Cu") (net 1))
 (via (at 206.75 158.4) (size 0.5) (drill 0.25) (layers "F.Cu" "B.Cu") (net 1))
 (via (at 205.35 154.15) (size 0.5) (drill 0.25) (layers "F.Cu" "B.Cu") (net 1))
 (via (at 214.83 150.62) (size 0.5) (drill 0.25) (layers "F.Cu" "B.Cu") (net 1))
 (segment (start 210.99 150.65) (end 211.5 151.16) (width 0.2) (layer "F.Cu") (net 3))
 (segment (start 210.99 150.625) (end 210.99 150.65) (width 0.2) (layer "F.Cu") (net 3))
 (segment (start 211.5 151.16) (end 211.5 152.35) (width 0.2) (layer "F.Cu") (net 3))
 (segment (start 214 158.19) (end 214.47 158.66) (width 0.2) (layer "F.Cu") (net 7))
 (segment (start 214.47 158.66) (end 217.41 158.66) (width 0.2) (layer "F.Cu") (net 7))
 (segment (start 217.41 158.66) (end 217.5 158.75) (width 0.2) (layer "F.Cu") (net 7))
 (segment (start 205.49 156.43) (end 205.25 156.67) (width 0.2) (layer "F.Cu") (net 6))
 (segment (start 205.49 156.3) (end 205.49 156.43) (width 0.2) (layer "F.Cu") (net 6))
 (segment (start 205.25 156.67) (end 205.25 157.4625) (width 0.2) (layer "F.Cu") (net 6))
 (segment (start 213.29 150.625) (end 213.29 150.65) (width 0.2) (layer "F.Cu") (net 2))
 (segment (start 213.29 150.625) (end 212.01 150.625) (width 0.2) (layer "F.Cu") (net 2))
 (segment (start 213.8 151.16) (end 213.8 152.35) (width 0.2) (layer "F.Cu") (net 2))
 (segment (start 213.29 150.65) (end 213.8 151.16) (width 0.2) (layer "F.Cu") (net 2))
 (segment (start 214.57 159.21) (end 214 159.21) (width 0.4) (layer "F.Cu") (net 5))
 (via (at 214.57 159.21) (size 0.5) (drill 0.25) (layers "F.Cu" "B.Cu") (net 5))
 (segment (start 214.33 159.45) (end 202.7 159.45) (width 0.4) (layer "B.Cu") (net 5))
 (segment (start 214.57 159.21) (end 214.33 159.45) (width 0.4) (layer "B.Cu") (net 5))
 (segment (start 202.7 159.45) (end 202 158.75) (width 0.4) (layer "B.Cu") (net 5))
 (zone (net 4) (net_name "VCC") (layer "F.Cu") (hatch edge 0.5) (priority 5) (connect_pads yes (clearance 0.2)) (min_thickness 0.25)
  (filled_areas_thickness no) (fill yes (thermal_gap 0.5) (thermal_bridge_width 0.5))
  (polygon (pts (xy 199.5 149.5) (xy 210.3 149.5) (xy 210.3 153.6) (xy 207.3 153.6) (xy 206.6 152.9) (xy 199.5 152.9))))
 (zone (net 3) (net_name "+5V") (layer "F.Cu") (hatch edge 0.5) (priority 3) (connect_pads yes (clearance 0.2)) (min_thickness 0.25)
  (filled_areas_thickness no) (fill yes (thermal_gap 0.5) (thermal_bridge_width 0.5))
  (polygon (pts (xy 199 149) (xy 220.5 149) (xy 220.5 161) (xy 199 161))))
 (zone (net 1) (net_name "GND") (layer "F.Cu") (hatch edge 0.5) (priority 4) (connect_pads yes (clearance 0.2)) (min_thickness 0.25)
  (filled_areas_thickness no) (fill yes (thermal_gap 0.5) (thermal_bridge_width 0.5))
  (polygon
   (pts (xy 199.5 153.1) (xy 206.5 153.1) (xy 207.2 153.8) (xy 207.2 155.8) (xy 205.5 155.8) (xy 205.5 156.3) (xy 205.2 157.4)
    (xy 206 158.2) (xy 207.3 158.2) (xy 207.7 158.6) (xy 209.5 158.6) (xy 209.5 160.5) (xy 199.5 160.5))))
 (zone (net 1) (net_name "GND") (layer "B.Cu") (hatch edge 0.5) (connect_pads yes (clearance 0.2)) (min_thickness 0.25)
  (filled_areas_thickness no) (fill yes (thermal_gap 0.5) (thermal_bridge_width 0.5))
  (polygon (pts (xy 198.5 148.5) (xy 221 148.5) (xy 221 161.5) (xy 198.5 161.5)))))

